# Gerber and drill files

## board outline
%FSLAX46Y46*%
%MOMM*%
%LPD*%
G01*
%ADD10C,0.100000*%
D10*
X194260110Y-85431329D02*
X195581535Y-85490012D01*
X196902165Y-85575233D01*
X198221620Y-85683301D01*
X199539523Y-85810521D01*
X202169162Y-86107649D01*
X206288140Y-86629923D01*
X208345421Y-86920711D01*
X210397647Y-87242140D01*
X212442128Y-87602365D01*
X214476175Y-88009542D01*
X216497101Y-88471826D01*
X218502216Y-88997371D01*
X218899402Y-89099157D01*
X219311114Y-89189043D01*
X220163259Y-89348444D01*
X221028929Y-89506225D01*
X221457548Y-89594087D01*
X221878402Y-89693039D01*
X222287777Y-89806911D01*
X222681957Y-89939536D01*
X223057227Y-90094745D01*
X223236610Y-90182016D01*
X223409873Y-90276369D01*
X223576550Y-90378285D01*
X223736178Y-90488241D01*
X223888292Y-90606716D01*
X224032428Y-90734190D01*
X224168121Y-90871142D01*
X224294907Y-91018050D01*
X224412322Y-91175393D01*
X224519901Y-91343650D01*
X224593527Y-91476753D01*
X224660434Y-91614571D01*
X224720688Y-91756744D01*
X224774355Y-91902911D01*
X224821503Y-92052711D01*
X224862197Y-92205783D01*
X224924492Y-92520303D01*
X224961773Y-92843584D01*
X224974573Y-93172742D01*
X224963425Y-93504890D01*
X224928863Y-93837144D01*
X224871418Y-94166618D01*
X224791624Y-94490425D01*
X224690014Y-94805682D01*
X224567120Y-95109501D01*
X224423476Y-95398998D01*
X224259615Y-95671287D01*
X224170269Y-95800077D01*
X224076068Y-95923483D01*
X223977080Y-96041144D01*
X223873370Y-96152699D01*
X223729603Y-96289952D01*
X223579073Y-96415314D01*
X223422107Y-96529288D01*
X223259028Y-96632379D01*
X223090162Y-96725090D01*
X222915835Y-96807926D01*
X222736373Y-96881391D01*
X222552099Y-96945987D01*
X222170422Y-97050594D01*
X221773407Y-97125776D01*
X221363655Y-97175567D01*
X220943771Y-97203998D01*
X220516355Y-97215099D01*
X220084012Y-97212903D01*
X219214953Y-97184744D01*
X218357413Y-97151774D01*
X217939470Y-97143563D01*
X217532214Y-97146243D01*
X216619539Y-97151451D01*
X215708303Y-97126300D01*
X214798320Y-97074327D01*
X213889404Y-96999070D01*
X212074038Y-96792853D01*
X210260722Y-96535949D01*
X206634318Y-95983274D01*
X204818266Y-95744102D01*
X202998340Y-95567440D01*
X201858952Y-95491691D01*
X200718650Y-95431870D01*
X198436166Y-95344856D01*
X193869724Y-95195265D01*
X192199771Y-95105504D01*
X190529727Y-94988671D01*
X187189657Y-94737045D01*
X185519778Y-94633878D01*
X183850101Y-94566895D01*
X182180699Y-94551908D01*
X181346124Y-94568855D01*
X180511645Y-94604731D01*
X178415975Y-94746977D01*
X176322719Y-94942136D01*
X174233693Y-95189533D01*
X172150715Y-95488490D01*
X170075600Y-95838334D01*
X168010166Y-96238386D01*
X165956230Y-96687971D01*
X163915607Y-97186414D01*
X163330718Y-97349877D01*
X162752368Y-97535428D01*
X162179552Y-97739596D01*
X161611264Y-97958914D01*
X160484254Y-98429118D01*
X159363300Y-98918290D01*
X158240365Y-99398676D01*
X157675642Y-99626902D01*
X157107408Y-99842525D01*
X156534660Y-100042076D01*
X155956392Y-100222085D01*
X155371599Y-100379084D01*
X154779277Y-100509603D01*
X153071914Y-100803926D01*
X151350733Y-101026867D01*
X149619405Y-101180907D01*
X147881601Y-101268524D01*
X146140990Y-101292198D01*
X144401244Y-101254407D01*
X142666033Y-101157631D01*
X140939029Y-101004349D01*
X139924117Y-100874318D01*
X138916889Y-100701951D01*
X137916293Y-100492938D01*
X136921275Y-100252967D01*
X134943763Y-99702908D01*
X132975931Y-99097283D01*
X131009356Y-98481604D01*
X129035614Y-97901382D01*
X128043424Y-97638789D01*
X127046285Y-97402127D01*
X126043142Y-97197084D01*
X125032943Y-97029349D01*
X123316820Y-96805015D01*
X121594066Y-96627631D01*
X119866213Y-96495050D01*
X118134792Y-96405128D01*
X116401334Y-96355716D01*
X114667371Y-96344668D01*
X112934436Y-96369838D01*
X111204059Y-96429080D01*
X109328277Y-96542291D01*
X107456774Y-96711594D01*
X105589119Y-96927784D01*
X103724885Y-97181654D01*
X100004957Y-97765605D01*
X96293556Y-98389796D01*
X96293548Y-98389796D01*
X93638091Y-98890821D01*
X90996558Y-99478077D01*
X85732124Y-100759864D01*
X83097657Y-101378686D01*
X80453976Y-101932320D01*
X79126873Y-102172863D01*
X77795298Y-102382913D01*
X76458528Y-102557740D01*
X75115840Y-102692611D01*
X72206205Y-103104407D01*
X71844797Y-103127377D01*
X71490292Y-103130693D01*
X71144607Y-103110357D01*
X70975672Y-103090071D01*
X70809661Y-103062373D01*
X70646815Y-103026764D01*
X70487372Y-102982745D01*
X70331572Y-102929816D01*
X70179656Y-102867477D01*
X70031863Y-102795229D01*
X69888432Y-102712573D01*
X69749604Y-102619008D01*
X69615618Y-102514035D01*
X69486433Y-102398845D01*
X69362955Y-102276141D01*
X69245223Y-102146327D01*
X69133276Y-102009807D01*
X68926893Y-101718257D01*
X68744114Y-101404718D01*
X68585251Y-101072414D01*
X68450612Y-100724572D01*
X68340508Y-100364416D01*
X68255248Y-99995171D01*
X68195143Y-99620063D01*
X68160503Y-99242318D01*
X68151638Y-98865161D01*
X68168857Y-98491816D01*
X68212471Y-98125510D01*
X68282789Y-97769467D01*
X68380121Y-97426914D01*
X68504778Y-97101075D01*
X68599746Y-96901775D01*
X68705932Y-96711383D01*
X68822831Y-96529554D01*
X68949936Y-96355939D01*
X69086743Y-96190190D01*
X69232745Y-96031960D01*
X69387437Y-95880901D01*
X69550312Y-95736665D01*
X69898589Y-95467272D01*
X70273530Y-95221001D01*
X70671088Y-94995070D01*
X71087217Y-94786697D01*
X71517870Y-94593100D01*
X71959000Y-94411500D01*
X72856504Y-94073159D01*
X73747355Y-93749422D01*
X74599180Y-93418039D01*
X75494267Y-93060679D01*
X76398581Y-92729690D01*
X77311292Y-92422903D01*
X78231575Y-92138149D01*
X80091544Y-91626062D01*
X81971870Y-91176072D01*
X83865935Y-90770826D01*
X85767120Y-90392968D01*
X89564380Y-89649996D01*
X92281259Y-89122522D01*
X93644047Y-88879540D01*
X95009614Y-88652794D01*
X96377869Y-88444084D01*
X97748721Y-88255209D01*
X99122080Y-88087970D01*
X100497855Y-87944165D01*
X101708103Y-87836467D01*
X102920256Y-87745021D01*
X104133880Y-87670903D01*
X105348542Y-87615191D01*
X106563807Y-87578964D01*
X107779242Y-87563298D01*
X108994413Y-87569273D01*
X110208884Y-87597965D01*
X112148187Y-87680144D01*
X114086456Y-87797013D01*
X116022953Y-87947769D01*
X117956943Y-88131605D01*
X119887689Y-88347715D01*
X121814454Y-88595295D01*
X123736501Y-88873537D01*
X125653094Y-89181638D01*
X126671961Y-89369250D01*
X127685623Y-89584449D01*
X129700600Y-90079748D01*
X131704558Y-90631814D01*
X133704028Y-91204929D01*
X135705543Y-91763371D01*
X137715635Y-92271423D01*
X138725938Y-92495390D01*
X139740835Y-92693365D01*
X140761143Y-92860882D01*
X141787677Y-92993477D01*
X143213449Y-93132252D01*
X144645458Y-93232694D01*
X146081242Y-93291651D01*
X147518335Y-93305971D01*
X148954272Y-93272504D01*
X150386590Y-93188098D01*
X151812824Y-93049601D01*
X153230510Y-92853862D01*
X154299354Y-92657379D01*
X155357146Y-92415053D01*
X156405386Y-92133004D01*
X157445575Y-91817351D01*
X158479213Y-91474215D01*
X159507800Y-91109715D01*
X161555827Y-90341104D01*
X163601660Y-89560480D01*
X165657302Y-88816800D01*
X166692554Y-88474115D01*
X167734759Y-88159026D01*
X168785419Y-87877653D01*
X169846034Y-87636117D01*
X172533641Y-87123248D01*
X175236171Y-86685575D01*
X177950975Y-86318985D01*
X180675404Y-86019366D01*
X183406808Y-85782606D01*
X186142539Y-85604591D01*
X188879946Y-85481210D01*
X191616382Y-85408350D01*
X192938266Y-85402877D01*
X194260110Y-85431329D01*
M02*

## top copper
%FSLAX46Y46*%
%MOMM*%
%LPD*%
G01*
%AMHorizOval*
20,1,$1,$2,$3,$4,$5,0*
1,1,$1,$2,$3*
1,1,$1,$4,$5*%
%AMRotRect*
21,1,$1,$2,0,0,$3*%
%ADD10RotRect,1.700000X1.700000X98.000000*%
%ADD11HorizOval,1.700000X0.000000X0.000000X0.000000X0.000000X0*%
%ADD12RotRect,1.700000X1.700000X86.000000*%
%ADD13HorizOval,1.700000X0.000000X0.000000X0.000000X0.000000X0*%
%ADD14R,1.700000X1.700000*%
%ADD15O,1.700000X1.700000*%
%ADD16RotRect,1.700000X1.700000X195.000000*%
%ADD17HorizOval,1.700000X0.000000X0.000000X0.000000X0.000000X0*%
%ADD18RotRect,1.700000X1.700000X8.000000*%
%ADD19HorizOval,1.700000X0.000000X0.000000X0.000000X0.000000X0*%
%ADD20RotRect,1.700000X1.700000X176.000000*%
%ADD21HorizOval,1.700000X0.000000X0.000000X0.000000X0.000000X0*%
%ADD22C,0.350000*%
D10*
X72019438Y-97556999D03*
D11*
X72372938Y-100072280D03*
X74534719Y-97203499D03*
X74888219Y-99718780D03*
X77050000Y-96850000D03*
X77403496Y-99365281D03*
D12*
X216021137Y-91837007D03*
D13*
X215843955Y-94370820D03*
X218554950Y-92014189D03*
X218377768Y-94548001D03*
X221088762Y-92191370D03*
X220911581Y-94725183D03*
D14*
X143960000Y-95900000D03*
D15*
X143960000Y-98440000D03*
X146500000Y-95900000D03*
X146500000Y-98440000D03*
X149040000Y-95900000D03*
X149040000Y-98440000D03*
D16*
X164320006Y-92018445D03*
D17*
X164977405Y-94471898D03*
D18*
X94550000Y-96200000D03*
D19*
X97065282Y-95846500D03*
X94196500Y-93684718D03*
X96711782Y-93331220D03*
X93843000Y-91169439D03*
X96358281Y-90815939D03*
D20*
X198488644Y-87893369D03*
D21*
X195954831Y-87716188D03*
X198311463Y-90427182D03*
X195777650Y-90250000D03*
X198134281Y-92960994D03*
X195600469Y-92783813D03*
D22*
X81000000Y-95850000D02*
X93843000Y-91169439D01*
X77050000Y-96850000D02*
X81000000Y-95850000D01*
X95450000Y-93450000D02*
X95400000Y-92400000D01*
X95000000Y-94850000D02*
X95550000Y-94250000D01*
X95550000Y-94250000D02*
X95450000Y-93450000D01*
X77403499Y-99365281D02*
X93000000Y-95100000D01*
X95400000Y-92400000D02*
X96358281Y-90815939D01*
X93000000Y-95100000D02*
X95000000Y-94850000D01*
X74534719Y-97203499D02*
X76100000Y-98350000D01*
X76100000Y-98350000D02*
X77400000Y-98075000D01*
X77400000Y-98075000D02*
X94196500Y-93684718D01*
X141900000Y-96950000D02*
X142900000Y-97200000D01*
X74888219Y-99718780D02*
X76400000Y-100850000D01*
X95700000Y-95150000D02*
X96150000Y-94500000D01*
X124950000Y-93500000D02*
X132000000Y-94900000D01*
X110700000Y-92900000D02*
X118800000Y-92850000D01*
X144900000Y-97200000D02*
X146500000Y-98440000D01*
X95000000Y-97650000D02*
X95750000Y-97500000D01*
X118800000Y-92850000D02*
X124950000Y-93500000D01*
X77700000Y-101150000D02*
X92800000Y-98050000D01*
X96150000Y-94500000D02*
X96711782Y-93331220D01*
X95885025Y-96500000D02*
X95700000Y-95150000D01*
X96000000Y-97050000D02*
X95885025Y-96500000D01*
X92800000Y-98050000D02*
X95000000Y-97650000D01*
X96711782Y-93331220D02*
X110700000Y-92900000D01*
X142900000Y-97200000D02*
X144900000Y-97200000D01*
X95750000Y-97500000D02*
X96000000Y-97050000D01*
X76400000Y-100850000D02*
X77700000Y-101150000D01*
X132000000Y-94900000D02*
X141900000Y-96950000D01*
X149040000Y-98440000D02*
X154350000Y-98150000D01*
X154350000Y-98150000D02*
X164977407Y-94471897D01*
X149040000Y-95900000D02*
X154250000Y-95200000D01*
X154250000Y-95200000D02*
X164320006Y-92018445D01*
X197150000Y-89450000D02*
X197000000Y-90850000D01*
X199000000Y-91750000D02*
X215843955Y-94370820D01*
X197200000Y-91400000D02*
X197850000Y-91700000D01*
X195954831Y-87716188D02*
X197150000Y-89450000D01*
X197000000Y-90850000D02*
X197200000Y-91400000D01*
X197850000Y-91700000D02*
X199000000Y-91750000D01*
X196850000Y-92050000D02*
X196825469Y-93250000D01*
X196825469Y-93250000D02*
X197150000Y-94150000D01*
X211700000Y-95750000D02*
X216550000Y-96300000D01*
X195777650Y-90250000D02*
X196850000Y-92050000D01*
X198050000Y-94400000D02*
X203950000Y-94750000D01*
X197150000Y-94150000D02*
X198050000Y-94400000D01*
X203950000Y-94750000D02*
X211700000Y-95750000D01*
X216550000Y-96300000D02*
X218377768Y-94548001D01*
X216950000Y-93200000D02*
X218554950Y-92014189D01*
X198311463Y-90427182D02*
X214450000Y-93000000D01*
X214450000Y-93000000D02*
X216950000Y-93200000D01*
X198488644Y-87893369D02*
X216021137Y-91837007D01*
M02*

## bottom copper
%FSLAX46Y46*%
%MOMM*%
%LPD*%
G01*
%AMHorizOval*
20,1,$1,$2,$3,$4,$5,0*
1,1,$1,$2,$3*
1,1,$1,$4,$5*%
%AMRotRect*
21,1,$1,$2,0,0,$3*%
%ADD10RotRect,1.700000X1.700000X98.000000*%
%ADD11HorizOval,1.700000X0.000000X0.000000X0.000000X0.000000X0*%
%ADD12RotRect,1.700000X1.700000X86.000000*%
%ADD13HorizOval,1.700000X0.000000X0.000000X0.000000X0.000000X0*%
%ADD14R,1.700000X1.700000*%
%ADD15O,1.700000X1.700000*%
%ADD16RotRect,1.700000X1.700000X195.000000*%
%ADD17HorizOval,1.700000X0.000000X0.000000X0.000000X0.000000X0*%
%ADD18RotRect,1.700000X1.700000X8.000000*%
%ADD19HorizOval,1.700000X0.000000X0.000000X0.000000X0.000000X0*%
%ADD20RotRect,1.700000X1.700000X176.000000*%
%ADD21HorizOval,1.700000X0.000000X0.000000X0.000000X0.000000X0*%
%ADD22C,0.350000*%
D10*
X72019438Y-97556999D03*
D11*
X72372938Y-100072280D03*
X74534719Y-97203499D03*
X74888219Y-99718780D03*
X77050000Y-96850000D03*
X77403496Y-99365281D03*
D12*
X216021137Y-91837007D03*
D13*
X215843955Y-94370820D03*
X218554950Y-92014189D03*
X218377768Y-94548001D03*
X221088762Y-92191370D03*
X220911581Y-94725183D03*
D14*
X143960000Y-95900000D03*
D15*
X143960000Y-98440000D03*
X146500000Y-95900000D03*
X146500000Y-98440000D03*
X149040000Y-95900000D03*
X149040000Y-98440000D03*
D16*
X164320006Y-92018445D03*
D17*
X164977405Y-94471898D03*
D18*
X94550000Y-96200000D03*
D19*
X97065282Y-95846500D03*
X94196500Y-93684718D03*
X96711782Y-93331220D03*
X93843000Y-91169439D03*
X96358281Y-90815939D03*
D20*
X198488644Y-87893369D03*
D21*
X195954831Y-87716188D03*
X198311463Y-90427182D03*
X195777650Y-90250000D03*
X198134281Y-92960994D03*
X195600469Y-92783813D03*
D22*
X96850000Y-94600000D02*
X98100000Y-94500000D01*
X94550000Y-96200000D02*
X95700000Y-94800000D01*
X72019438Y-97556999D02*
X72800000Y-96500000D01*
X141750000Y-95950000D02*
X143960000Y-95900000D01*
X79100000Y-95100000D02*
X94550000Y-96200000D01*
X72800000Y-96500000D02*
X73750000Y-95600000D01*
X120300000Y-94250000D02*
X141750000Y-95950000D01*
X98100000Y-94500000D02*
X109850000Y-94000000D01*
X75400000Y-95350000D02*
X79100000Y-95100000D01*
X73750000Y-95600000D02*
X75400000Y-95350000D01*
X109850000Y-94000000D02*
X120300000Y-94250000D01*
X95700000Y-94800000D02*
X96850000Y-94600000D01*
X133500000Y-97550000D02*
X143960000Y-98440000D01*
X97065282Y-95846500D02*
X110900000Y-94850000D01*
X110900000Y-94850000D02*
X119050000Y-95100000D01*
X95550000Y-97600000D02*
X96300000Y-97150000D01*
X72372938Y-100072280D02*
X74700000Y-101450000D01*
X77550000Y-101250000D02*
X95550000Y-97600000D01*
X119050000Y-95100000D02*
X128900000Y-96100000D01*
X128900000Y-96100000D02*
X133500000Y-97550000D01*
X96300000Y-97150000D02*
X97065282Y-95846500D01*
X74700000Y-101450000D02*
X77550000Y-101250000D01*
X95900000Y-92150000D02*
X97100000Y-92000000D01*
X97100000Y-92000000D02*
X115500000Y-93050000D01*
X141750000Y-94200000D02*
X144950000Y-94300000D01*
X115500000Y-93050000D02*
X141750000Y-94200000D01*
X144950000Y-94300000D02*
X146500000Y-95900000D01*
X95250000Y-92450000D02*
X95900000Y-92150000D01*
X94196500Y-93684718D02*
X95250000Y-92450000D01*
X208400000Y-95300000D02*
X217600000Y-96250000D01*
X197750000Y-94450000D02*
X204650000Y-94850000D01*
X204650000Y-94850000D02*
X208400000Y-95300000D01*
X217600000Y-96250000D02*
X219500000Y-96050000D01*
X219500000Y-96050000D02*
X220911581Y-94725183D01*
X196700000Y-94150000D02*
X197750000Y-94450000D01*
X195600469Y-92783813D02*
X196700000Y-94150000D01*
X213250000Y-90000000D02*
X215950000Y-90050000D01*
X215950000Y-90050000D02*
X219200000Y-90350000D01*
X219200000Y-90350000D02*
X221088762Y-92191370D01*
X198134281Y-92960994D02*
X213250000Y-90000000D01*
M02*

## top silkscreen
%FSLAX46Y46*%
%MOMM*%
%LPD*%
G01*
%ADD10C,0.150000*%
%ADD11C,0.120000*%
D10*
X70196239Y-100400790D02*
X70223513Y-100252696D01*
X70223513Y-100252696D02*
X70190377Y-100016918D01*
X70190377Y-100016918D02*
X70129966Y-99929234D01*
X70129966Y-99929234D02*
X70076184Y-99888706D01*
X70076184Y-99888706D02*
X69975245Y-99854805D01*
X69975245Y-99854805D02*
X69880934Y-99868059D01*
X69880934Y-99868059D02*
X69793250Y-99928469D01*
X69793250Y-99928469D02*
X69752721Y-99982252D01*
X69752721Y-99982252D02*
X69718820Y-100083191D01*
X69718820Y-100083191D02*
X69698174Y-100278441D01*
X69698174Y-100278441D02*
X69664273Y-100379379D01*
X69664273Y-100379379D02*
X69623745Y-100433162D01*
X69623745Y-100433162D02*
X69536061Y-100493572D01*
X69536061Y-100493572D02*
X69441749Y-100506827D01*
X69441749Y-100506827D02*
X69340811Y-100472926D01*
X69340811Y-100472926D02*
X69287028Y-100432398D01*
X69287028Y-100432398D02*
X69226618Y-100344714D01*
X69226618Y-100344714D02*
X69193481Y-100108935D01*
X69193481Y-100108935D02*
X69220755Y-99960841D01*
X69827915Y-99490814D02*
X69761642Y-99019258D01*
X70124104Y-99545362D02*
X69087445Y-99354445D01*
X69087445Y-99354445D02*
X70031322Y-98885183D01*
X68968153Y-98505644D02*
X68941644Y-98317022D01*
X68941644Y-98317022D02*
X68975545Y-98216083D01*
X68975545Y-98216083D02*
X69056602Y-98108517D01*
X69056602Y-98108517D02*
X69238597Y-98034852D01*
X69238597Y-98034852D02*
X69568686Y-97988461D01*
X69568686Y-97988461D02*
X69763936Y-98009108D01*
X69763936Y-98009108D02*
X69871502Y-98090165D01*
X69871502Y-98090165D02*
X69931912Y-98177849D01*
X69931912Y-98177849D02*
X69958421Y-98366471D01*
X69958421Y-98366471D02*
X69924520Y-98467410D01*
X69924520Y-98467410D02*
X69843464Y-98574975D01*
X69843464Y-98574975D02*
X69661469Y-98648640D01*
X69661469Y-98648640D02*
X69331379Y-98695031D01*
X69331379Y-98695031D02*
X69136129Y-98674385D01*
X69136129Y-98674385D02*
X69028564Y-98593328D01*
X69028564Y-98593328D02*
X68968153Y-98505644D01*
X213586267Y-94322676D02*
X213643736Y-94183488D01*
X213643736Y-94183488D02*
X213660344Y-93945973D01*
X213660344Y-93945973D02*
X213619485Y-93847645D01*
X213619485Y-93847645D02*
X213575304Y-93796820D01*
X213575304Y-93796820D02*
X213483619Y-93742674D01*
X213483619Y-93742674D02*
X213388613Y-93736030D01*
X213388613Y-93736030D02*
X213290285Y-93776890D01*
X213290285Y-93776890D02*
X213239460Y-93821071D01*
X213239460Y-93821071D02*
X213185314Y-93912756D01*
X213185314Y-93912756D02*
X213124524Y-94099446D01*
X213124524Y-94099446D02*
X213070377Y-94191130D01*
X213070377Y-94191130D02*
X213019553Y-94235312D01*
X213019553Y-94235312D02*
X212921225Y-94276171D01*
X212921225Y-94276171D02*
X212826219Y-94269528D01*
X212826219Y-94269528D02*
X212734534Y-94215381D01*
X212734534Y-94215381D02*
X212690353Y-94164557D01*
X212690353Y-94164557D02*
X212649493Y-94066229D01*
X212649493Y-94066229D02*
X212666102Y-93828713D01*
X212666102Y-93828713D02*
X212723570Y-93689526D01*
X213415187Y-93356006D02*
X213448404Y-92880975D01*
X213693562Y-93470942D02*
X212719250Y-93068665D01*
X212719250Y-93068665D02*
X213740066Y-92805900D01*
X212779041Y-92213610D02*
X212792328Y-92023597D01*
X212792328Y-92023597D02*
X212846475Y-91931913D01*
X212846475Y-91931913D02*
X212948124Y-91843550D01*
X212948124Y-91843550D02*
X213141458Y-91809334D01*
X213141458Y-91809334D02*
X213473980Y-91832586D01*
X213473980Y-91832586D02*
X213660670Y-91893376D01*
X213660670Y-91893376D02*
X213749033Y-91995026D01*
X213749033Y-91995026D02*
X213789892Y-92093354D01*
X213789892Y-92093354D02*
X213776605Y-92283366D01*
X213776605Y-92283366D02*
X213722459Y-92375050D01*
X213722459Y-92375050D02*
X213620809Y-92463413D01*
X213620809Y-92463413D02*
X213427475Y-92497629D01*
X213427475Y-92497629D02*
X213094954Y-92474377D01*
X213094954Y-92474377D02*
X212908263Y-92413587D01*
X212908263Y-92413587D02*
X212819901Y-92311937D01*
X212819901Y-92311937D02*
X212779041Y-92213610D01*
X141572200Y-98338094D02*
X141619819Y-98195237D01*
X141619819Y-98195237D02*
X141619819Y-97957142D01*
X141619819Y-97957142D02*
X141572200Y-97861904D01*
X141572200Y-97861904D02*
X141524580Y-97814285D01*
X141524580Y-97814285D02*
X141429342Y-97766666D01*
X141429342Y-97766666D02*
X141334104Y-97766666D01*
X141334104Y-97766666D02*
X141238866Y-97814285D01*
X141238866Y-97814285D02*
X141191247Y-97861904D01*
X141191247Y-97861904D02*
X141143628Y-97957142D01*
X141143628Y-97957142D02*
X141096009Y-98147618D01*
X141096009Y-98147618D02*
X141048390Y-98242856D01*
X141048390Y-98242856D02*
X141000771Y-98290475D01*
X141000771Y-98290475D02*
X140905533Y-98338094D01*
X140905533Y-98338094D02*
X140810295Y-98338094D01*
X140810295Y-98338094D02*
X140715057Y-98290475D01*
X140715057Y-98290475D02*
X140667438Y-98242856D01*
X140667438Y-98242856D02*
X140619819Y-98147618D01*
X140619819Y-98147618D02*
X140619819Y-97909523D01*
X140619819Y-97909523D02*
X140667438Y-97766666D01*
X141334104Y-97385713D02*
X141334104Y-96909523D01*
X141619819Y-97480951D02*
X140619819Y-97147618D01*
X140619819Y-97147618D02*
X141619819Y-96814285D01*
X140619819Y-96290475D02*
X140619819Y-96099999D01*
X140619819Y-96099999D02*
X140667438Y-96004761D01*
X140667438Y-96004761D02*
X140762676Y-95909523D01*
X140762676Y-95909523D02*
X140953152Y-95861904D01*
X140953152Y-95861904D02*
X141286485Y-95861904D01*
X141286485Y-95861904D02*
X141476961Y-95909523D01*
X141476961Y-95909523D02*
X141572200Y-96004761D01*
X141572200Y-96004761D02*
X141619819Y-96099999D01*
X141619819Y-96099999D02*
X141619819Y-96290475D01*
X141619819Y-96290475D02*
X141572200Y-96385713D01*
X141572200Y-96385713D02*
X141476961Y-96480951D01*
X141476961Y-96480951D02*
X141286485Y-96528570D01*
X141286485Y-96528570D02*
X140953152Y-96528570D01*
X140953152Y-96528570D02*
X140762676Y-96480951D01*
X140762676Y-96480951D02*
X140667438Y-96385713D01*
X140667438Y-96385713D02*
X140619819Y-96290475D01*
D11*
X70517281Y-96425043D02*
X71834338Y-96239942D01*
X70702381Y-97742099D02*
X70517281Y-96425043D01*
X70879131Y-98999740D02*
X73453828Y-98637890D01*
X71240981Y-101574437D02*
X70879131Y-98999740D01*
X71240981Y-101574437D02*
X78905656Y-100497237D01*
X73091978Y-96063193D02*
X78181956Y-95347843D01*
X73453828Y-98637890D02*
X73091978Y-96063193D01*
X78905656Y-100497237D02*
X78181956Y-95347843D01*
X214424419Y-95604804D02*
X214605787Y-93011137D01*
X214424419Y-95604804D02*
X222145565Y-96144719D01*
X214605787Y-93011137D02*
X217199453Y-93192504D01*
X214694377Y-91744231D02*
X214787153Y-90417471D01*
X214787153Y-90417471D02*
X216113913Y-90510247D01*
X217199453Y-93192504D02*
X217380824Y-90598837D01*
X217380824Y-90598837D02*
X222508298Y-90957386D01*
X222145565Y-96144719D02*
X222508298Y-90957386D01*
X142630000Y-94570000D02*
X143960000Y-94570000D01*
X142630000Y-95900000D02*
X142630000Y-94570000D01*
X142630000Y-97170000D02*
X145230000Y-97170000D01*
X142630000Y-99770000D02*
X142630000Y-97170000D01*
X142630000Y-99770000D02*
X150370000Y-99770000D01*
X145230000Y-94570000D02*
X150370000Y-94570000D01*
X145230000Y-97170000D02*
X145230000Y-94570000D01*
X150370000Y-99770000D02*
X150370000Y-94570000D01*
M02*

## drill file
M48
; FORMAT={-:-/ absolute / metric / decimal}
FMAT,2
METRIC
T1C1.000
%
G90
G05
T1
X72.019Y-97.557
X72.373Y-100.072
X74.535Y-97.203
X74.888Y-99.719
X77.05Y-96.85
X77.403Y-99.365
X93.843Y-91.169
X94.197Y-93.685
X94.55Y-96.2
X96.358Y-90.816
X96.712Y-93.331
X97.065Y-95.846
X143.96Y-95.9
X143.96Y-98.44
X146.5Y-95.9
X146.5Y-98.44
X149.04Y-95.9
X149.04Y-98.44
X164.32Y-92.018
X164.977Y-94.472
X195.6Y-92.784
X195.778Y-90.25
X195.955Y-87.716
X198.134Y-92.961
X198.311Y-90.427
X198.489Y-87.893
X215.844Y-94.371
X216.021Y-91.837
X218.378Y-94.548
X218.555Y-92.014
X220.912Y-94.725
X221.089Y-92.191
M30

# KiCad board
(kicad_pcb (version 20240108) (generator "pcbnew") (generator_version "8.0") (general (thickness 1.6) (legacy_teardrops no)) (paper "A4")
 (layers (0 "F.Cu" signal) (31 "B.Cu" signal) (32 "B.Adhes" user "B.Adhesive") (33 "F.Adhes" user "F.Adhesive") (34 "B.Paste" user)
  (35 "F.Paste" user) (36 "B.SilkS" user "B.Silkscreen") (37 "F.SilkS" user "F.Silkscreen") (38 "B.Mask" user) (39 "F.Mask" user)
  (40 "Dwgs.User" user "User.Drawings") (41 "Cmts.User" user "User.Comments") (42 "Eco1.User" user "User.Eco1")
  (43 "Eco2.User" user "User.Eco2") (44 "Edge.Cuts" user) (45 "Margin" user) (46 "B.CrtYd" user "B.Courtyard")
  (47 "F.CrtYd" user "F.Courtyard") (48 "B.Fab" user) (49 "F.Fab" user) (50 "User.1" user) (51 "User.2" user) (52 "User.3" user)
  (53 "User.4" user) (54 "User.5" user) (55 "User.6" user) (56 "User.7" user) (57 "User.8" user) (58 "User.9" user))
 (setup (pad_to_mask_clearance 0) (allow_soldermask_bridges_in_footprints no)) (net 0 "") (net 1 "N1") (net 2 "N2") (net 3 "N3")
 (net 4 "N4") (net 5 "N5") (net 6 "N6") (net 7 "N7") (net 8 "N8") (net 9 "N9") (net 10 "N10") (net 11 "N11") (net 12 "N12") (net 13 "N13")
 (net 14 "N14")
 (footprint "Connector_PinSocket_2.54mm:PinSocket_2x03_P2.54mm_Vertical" (layer "F.Cu") (at 72.019438 97.556999 98)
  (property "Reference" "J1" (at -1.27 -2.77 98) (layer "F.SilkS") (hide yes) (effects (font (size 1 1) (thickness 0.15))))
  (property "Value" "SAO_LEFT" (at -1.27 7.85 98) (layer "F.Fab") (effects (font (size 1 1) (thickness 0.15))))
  (fp_line (start 1.33 -1.33) (end 1.33 0) (stroke (width 0.12) (type solid)) (layer "F.SilkS"))
  (fp_line (start 0 -1.33) (end 1.33 -1.33) (stroke (width 0.12) (type solid)) (layer "F.SilkS"))
  (fp_line (start -1.27 -1.33) (end -1.27 1.27) (stroke (width 0.12) (type solid)) (layer "F.SilkS"))
  (fp_line (start -3.87 -1.33) (end -1.27 -1.33) (stroke (width 0.12) (type solid)) (layer "F.SilkS"))
  (fp_line (start -3.87 -1.33) (end -3.87 6.41) (stroke (width 0.12) (type solid)) (layer "F.SilkS"))
  (fp_line (start 1.33 1.27) (end 1.33 6.41) (stroke (width 0.12) (type solid)) (layer "F.SilkS"))
  (fp_line (start -1.27 1.27) (end 1.33 1.27) (stroke (width 0.12) (type solid)) (layer "F.SilkS"))
  (fp_line (start -3.87 6.41) (end 1.33 6.41) (stroke (width 0.12) (type solid)) (layer "F.SilkS"))
  (pad "1" thru_hole rect (at 0 0 98) (size 1.7 1.7) (drill 1) (layers "*.Cu" "*.Mask") (remove_unused_layers no) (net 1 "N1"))
  (pad "2" thru_hole oval (at -2.54 0 98) (size 1.7 1.7) (drill 1) (layers "*.Cu" "*.Mask") (remove_unused_layers no) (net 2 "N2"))
  (pad "3" thru_hole oval (at 0 2.54 98) (size 1.7 1.7) (drill 1) (layers "*.Cu" "*.Mask") (remove_unused_layers no) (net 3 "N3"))
  (pad "4" thru_hole oval (at -2.54 2.54 98) (size 1.7 1.7) (drill 1) (layers "*.Cu" "*.Mask") (remove_unused_layers no) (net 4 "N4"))
  (pad "5" thru_hole oval (at 0 5.08 98) (size 1.7 1.7) (drill 1) (layers "*.Cu" "*.Mask") (remove_unused_layers no) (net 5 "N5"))
  (pad "6" thru_hole oval (at -2.54 5.079997 98) (size 1.7 1.7) (drill 1) (layers "*.Cu" "*.Mask") (remove_unused_layers no) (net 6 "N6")))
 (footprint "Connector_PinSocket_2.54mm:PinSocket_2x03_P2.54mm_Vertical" (layer "F.Cu") (at 216.021137 91.837007 86)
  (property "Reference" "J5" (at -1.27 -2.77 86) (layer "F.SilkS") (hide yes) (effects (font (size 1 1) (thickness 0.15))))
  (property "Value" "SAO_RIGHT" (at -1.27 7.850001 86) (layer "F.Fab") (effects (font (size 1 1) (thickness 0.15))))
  (fp_line (start -3.87 -1.33) (end -1.27 -1.329999) (stroke (width 0.12) (type solid)) (layer "F.SilkS"))
  (fp_line (start -3.87 -1.33) (end -3.87 6.41) (stroke (width 0.12) (type solid)) (layer "F.SilkS"))
  (fp_line (start -1.27 -1.329999) (end -1.27 1.27) (stroke (width 0.12) (type solid)) (layer "F.SilkS"))
  (fp_line (start 0 -1.33) (end 1.33 -1.33) (stroke (width 0.12) (type solid)) (layer "F.SilkS"))
  (fp_line (start 1.33 -1.33) (end 1.33 0) (stroke (width 0.12) (type solid)) (layer "F.SilkS"))
  (fp_line (start -1.27 1.27) (end 1.330001 1.270004) (stroke (width 0.12) (type solid)) (layer "F.SilkS"))
  (fp_line (start 1.330001 1.270004) (end 1.33 6.409999) (stroke (width 0.12) (type solid)) (layer "F.SilkS"))
  (fp_line (start -3.87 6.41) (end 1.33 6.409999) (stroke (width 0.12) (type solid)) (layer "F.SilkS"))
  (pad "1" thru_hole rect (at 0 0 86) (size 1.7 1.7) (drill 1) (layers "*.Cu" "*.Mask") (remove_unused_layers no) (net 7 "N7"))
  (pad "2" thru_hole oval (at -2.54 -0.000001 86) (size 1.7 1.7) (drill 1) (layers "*.Cu" "*.Mask") (remove_unused_layers no) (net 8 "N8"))
  (pad "3" thru_hole oval (at -0.000001 2.54 86) (size 1.7 1.7) (drill 1) (layers "*.Cu" "*.Mask") (remove_unused_layers no) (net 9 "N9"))
  (pad "4" thru_hole oval (at -2.54 2.54 86) (size 1.7 1.7) (drill 1) (layers "*.Cu" "*.Mask") (remove_unused_layers no) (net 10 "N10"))
  (pad "5" thru_hole oval (at 0 5.08 86) (size 1.7 1.7) (drill 1) (layers "*.Cu" "*.Mask") (remove_unused_layers no) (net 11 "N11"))
  (pad "6" thru_hole oval (at -2.54 5.08 86) (size 1.7 1.7) (drill 1) (layers "*.Cu" "*.Mask") (remove_unused_layers no) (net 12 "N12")))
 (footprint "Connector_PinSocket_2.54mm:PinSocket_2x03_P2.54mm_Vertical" (layer "F.Cu") (at 143.96 95.9 90)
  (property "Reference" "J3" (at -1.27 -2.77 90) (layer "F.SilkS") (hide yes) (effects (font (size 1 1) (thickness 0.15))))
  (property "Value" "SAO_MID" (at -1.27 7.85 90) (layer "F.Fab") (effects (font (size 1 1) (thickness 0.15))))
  (fp_line (start 1.33 -1.33) (end 1.33 0) (stroke (width 0.12) (type solid)) (layer "F.SilkS"))
  (fp_line (start 0 -1.33) (end 1.33 -1.33) (stroke (width 0.12) (type solid)) (layer "F.SilkS"))
  (fp_line (start -1.27 -1.33) (end -1.27 1.27) (stroke (width 0.12) (type solid)) (layer "F.SilkS"))
  (fp_line (start -3.87 -1.33) (end -1.27 -1.33) (stroke (width 0.12) (type solid)) (layer "F.SilkS"))
  (fp_line (start -3.87 -1.33) (end -3.87 6.41) (stroke (width 0.12) (type solid)) (layer "F.SilkS"))
  (fp_line (start 1.33 1.27) (end 1.33 6.41) (stroke (width 0.12) (type solid)) (layer "F.SilkS"))
  (fp_line (start -1.27 1.27) (end 1.33 1.27) (stroke (width 0.12) (type solid)) (layer "F.SilkS"))
  (fp_line (start -3.87 6.41) (end 1.33 6.41) (stroke (width 0.12) (type solid)) (layer "F.SilkS"))
  (pad "1" thru_hole rect (at 0 0 90) (size 1.7 1.7) (drill 1) (layers "*.Cu" "*.Mask") (remove_unused_layers no) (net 1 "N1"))
  (pad "2" thru_hole oval (at -2.54 0 90) (size 1.7 1.7) (drill 1) (layers "*.Cu" "*.Mask") (remove_unused_layers no) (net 2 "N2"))
  (pad "3" thru_hole oval (at 0 2.54 90) (size 1.7 1.7) (drill 1) (layers "*.Cu" "*.Mask") (remove_unused_layers no) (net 3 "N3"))
  (pad "4" thru_hole oval (at -2.54 2.54 90) (size 1.7 1.7) (drill 1) (layers "*.Cu" "*.Mask") (remove_unused_layers no) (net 4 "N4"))
  (pad "5" thru_hole oval (at 0 5.08 90) (size 1.7 1.7) (drill 1) (layers "*.Cu" "*.Mask") (remove_unused_layers no) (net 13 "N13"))
  (pad "6" thru_hole oval (at -2.54 5.08 90) (size 1.7 1.7) (drill 1) (layers "*.Cu" "*.Mask") (remove_unused_layers no) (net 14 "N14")))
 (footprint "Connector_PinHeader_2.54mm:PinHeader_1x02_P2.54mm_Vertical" (layer "B.Cu") (at 164.320006 92.018445 -165)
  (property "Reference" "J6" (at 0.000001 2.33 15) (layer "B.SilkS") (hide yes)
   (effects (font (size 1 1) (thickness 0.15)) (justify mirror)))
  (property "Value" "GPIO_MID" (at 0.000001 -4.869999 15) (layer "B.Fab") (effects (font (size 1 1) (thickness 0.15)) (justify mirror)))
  (pad "1" thru_hole rect (at 0 0 195) (size 1.7 1.7) (drill 1) (layers "*.Cu" "*.Mask") (remove_unused_layers no) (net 13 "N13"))
  (pad "2" thru_hole oval (at 0.000002 -2.540001 195) (size 1.7 1.7) (drill 1) (layers "*.Cu" "*.Mask") (remove_unused_layers no)
   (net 14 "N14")))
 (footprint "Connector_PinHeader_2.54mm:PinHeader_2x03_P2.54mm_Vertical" (layer "B.Cu") (at 94.55 96.2 8)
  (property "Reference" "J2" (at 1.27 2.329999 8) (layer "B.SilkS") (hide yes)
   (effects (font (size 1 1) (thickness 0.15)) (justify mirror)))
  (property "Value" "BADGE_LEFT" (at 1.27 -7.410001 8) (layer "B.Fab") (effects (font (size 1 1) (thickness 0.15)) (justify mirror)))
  (pad "1" thru_hole rect (at 0 0 8) (size 1.7 1.7) (drill 1) (layers "*.Cu" "*.Mask") (remove_unused_layers no) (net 1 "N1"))
  (pad "2" thru_hole oval (at 2.540001 0 8) (size 1.7 1.7) (drill 1) (layers "*.Cu" "*.Mask") (remove_unused_layers no) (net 2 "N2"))
  (pad "3" thru_hole oval (at 0 -2.540001 8) (size 1.7 1.7) (drill 1) (layers "*.Cu" "*.Mask") (remove_unused_layers no) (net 3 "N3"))
  (pad "4" thru_hole oval (at 2.540001 -2.539999 8) (size 1.7 1.7) (drill 1) (layers "*.Cu" "*.Mask") (remove_unused_layers no) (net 4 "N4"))
  (pad "5" thru_hole oval (at -0.000001 -5.079999 8) (size 1.7 1.7) (drill 1) (layers "*.Cu" "*.Mask") (remove_unused_layers no)
   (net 5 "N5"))
  (pad "6" thru_hole oval (at 2.539999 -5.08 8) (size 1.7 1.7) (drill 1) (layers "*.Cu" "*.Mask") (remove_unused_layers no) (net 6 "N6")))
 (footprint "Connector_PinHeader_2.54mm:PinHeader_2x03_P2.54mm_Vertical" (layer "B.Cu") (at 198.488644 87.893369 176)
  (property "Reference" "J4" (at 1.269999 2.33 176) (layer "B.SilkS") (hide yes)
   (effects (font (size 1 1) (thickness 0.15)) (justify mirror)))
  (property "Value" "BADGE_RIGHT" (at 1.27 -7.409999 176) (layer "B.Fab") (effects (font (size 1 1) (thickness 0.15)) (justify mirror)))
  (pad "1" thru_hole rect (at 0 0 176) (size 1.7 1.7) (drill 1) (layers "*.Cu" "*.Mask") (remove_unused_layers no) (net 7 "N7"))
  (pad "2" thru_hole oval (at 2.54 0 176) (size 1.7 1.7) (drill 1) (layers "*.Cu" "*.Mask") (remove_unused_layers no) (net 8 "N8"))
  (pad "3" thru_hole oval (at 0 -2.54 176) (size 1.7 1.7) (drill 1) (layers "*.Cu" "*.Mask") (remove_unused_layers no) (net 9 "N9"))
  (pad "4" thru_hole oval (at 2.54 -2.54 176) (size 1.7 1.7) (drill 1) (layers "*.Cu" "*.Mask") (remove_unused_layers no) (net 10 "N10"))
  (pad "5" thru_hole oval (at 0 -5.08 176) (size 1.7 1.7) (drill 1) (layers "*.Cu" "*.Mask") (remove_unused_layers no) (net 11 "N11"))
  (pad "6" thru_hole oval (at 2.539999 -5.08 176) (size 1.7 1.7) (drill 1) (layers "*.Cu" "*.Mask") (remove_unused_layers no) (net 12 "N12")))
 (gr_poly
  (pts (xy 194.26011 85.431329) (xy 195.581535 85.490012) (xy 196.902165 85.575233) (xy 198.22162 85.683301) (xy 199.539523 85.810521)
   (xy 202.169162 86.107649) (xy 206.28814 86.629923) (xy 208.345421 86.920711) (xy 210.397647 87.24214) (xy 212.442128 87.602365)
   (xy 214.476175 88.009542) (xy 216.497101 88.471826) (xy 218.502216 88.997371) (xy 218.899402 89.099157) (xy 219.311114 89.189043)
   (xy 220.163259 89.348444) (xy 221.028929 89.506225) (xy 221.457548 89.594087) (xy 221.878402 89.693039) (xy 222.287777 89.806911)
   (xy 222.681957 89.939536) (xy 223.057227 90.094745) (xy 223.23661 90.182016) (xy 223.409873 90.276369) (xy 223.57655 90.378285)
   (xy 223.736178 90.488241) (xy 223.888292 90.606716) (xy 224.032428 90.73419) (xy 224.168121 90.871142) (xy 224.294907 91.01805)
   (xy 224.412322 91.175393) (xy 224.519901 91.34365) (xy 224.593527 91.476753) (xy 224.660434 91.614571) (xy 224.720688 91.756744)
   (xy 224.774355 91.902911) (xy 224.821503 92.052711) (xy 224.862197 92.205783) (xy 224.924492 92.520303) (xy 224.961773 92.843584)
   (xy 224.974573 93.172742) (xy 224.963425 93.50489) (xy 224.928863 93.837144) (xy 224.871418 94.166618) (xy 224.791624 94.490425)
   (xy 224.690014 94.805682) (xy 224.56712 95.109501) (xy 224.423476 95.398998) (xy 224.259615 95.671287) (xy 224.170269 95.800077)
   (xy 224.076068 95.923483) (xy 223.97708 96.041144) (xy 223.87337 96.152699) (xy 223.729603 96.289952) (xy 223.579073 96.415314)
   (xy 223.422107 96.529288) (xy 223.259028 96.632379) (xy 223.090162 96.72509) (xy 222.915835 96.807926) (xy 222.736373 96.881391)
   (xy 222.552099 96.945987) (xy 222.170422 97.050594) (xy 221.773407 97.125776) (xy 221.363655 97.175567) (xy 220.943771 97.203998)
   (xy 220.516355 97.215099) (xy 220.084012 97.212903) (xy 219.214953 97.184744) (xy 218.357413 97.151774) (xy 217.93947 97.143563)
   (xy 217.532214 97.146243) (xy 216.619539 97.151451) (xy 215.708303 97.1263) (xy 214.79832 97.074327) (xy 213.889404 96.99907)
   (xy 212.074038 96.792853) (xy 210.260722 96.535949) (xy 206.634318 95.983274) (xy 204.818266 95.744102) (xy 202.99834 95.56744)
   (xy 201.858952 95.491691) (xy 200.71865 95.43187) (xy 198.436166 95.344856) (xy 193.869724 95.195265) (xy 192.199771 95.105504)
   (xy 190.529727 94.988671) (xy 187.189657 94.737045) (xy 185.519778 94.633878) (xy 183.850101 94.566895) (xy 182.180699 94.551908)
   (xy 181.346124 94.568855) (xy 180.511645 94.604731) (xy 178.415975 94.746977) (xy 176.322719 94.942136) (xy 174.233693 95.189533)
   (xy 172.150715 95.48849) (xy 170.0756 95.838334) (xy 168.010166 96.238386) (xy 165.95623 96.687971) (xy 163.915607 97.186414)
   (xy 163.330718 97.349877) (xy 162.752368 97.535428) (xy 162.179552 97.739596) (xy 161.611264 97.958914) (xy 160.484254 98.429118)
   (xy 159.3633 98.91829) (xy 158.240365 99.398676) (xy 157.675642 99.626902) (xy 157.107408 99.842525) (xy 156.53466 100.042076)
   (xy 155.956392 100.222085) (xy 155.371599 100.379084) (xy 154.779277 100.509603) (xy 153.071914 100.803926) (xy 151.350733 101.026867)
   (xy 149.619405 101.180907) (xy 147.881601 101.268524) (xy 146.14099 101.292198) (xy 144.401244 101.254407) (xy 142.666033 101.157631)
   (xy 140.939029 101.004349) (xy 139.924117 100.874318) (xy 138.916889 100.701951) (xy 137.916293 100.492938) (xy 136.921275 100.252967)
   (xy 134.943763 99.702908) (xy 132.975931 99.097283) (xy 131.009356 98.481604) (xy 129.035614 97.901382) (xy 128.043424 97.638789)
   (xy 127.046285 97.402127) (xy 126.043142 97.197084) (xy 125.032943 97.029349) (xy 123.31682 96.805015) (xy 121.594066 96.627631)
   (xy 119.866213 96.49505) (xy 118.134792 96.405128) (xy 116.401334 96.355716) (xy 114.667371 96.344668) (xy 112.934436 96.369838)
   (xy 111.204059 96.42908) (xy 109.328277 96.542291) (xy 107.456774 96.711594) (xy 105.589119 96.927784) (xy 103.724885 97.181654)
   (xy 100.004957 97.765605) (xy 96.293556 98.389796) (xy 96.293548 98.389796) (xy 93.638091 98.890821) (xy 90.996558 99.478077)
   (xy 85.732124 100.759864) (xy 83.097657 101.378686) (xy 80.453976 101.93232) (xy 79.126873 102.172863) (xy 77.795298 102.382913)
   (xy 76.458528 102.55774) (xy 75.11584 102.692611) (xy 72.206205 103.104407) (xy 71.844797 103.127377) (xy 71.490292 103.130693)
   (xy 71.144607 103.110357) (xy 70.975672 103.090071) (xy 70.809661 103.062373) (xy 70.646815 103.026764) (xy 70.487372 102.982745)
   (xy 70.331572 102.929816) (xy 70.179656 102.867477) (xy 70.031863 102.795229) (xy 69.888432 102.712573) (xy 69.749604 102.619008)
   (xy 69.615618 102.514035) (xy 69.486433 102.398845) (xy 69.362955 102.276141) (xy 69.245223 102.146327) (xy 69.133276 102.009807)
   (xy 68.926893 101.718257) (xy 68.744114 101.404718) (xy 68.585251 101.072414) (xy 68.450612 100.724572) (xy 68.340508 100.364416)
   (xy 68.255248 99.995171) (xy 68.195143 99.620063) (xy 68.160503 99.242318) (xy 68.151638 98.865161) (xy 68.168857 98.491816)
   (xy 68.212471 98.12551) (xy 68.282789 97.769467) (xy 68.380121 97.426914) (xy 68.504778 97.101075) (xy 68.599746 96.901775)
   (xy 68.705932 96.711383) (xy 68.822831 96.529554) (xy 68.949936 96.355939) (xy 69.086743 96.19019) (xy 69.232745 96.03196)
   (xy 69.387437 95.880901) (xy 69.550312 95.736665) (xy 69.898589 95.467272) (xy 70.27353 95.221001) (xy 70.671088 94.99507)
   (xy 71.087217 94.786697) (xy 71.51787 94.5931) (xy 71.959 94.4115) (xy 72.856504 94.073159) (xy 73.747355 93.749422)
   (xy 74.59918 93.418039) (xy 75.494267 93.060679) (xy 76.398581 92.72969) (xy 77.311292 92.422903) (xy 78.231575 92.138149)
   (xy 80.091544 91.626062) (xy 81.97187 91.176072) (xy 83.865935 90.770826) (xy 85.76712 90.392968) (xy 89.56438 89.649996)
   (xy 92.281259 89.122522) (xy 93.644047 88.87954) (xy 95.009614 88.652794) (xy 96.377869 88.444084) (xy 97.748721 88.255209)
   (xy 99.12208 88.08797) (xy 100.497855 87.944165) (xy 101.708103 87.836467) (xy 102.920256 87.745021) (xy 104.13388 87.670903)
   (xy 105.348542 87.615191) (xy 106.563807 87.578964) (xy 107.779242 87.563298) (xy 108.994413 87.569273) (xy 110.208884 87.597965)
   (xy 112.148187 87.680144) (xy 114.086456 87.797013) (xy 116.022953 87.947769) (xy 117.956943 88.131605) (xy 119.887689 88.347715)
   (xy 121.814454 88.595295) (xy 123.736501 88.873537) (xy 125.653094 89.181638) (xy 126.671961 89.36925) (xy 127.685623 89.584449)
   (xy 129.7006 90.079748) (xy 131.704558 90.631814) (xy 133.704028 91.204929) (xy 135.705543 91.763371) (xy 137.715635 92.271423)
   (xy 138.725938 92.49539) (xy 139.740835 92.693365) (xy 140.761143 92.860882) (xy 141.787677 92.993477) (xy 143.213449 93.132252)
   (xy 144.645458 93.232694) (xy 146.081242 93.291651) (xy 147.518335 93.305971) (xy 148.954272 93.272504) (xy 150.38659 93.188098)
   (xy 151.812824 93.049601) (xy 153.23051 92.853862) (xy 154.299354 92.657379) (xy 155.357146 92.415053) (xy 156.405386 92.133004)
   (xy 157.445575 91.817351) (xy 158.479213 91.474215) (xy 159.5078 91.109715) (xy 161.555827 90.341104) (xy 163.60166 89.56048)
   (xy 165.657302 88.8168) (xy 166.692554 88.474115) (xy 167.734759 88.159026) (xy 168.785419 87.877653) (xy 169.846034 87.636117)
   (xy 172.533641 87.123248) (xy 175.236171 86.685575) (xy 177.950975 86.318985) (xy 180.675404 86.019366) (xy 183.406808 85.782606)
   (xy 186.142539 85.604591) (xy 188.879946 85.48121) (xy 191.616382 85.40835) (xy 192.938266 85.402877))
  (stroke (width 0.1) (type solid)) (fill none) (layer "Edge.Cuts"))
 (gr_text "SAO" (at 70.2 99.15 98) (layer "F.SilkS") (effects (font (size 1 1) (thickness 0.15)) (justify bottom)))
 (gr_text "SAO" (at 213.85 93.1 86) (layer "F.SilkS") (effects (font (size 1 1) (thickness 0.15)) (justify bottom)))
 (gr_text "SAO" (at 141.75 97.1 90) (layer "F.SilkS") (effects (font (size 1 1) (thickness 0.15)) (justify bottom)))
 (segment (start 96.85 94.6) (end 98.1 94.5) (width 0.35) (layer "B.Cu") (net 1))
 (segment (start 94.55 96.2) (end 95.7 94.8) (width 0.35) (layer "B.Cu") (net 1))
 (segment (start 72.019438 97.556999) (end 72.8 96.5) (width 0.35) (layer "B.Cu") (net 1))
 (segment (start 141.75 95.95) (end 143.96 95.9) (width 0.35) (layer "B.Cu") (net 1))
 (segment (start 79.1 95.1) (end 94.55 96.2) (width 0.35) (layer "B.Cu") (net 1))
 (segment (start 72.8 96.5) (end 73.75 95.6) (width 0.35) (layer "B.Cu") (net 1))
 (segment (start 120.3 94.25) (end 141.75 95.95) (width 0.35) (layer "B.Cu") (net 1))
 (segment (start 98.1 94.5) (end 109.85 94) (width 0.35) (layer "B.Cu") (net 1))
 (segment (start 75.4 95.35) (end 79.1 95.1) (width 0.35) (layer "B.Cu") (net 1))
 (segment (start 73.75 95.6) (end 75.4 95.35) (width 0.35) (layer "B.Cu") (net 1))
 (segment (start 109.85 94) (end 120.3 94.25) (width 0.35) (layer "B.Cu") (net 1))
 (segment (start 95.7 94.8) (end 96.85 94.6) (width 0.35) (layer "B.Cu") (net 1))
 (segment (start 81 95.85) (end 93.843 91.169439) (width 0.35) (layer "F.Cu") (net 5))
 (segment (start 77.05 96.85) (end 81 95.85) (width 0.35) (layer "F.Cu") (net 5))
 (segment (start 95.45 93.45) (end 95.4 92.4) (width 0.35) (layer "F.Cu") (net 6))
 (segment (start 95 94.85) (end 95.55 94.25) (width 0.35) (layer "F.Cu") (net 6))
 (segment (start 95.55 94.25) (end 95.45 93.45) (width 0.35) (layer "F.Cu") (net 6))
 (segment (start 77.403499 99.365281) (end 93 95.1) (width 0.35) (layer "F.Cu") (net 6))
 (segment (start 95.4 92.4) (end 96.358281 90.815939) (width 0.35) (layer "F.Cu") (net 6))
 (segment (start 93 95.1) (end 95 94.85) (width 0.35) (layer "F.Cu") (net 6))
 (segment (start 133.5 97.55) (end 143.96 98.44) (width 0.35) (layer "B.Cu") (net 2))
 (segment (start 97.065282 95.8465) (end 110.9 94.85) (width 0.35) (layer "B.Cu") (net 2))
 (segment (start 110.9 94.85) (end 119.05 95.1) (width 0.35) (layer "B.Cu") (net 2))
 (segment (start 95.55 97.6) (end 96.3 97.15) (width 0.35) (layer "B.Cu") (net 2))
 (segment (start 72.372938 100.07228) (end 74.7 101.45) (width 0.35) (layer "B.Cu") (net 2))
 (segment (start 77.55 101.25) (end 95.55 97.6) (width 0.35) (layer "B.Cu") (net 2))
 (segment (start 119.05 95.1) (end 128.9 96.1) (width 0.35) (layer "B.Cu") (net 2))
 (segment (start 128.9 96.1) (end 133.5 97.55) (width 0.35) (layer "B.Cu") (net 2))
 (segment (start 96.3 97.15) (end 97.065282 95.8465) (width 0.35) (layer "B.Cu") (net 2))
 (segment (start 74.7 101.45) (end 77.55 101.25) (width 0.35) (layer "B.Cu") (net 2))
 (segment (start 74.534719 97.203499) (end 76.1 98.35) (width 0.35) (layer "F.Cu") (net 3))
 (segment (start 76.1 98.35) (end 77.4 98.075) (width 0.35) (layer "F.Cu") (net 3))
 (segment (start 77.4 98.075) (end 94.1965 93.684718) (width 0.35) (layer "F.Cu") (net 3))
 (segment (start 95.9 92.15) (end 97.1 92) (width 0.35) (layer "B.Cu") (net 3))
 (segment (start 97.1 92) (end 115.5 93.05) (width 0.35) (layer "B.Cu") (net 3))
 (segment (start 141.75 94.2) (end 144.95 94.3) (width 0.35) (layer "B.Cu") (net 3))
 (segment (start 115.5 93.05) (end 141.75 94.2) (width 0.35) (layer "B.Cu") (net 3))
 (segment (start 144.95 94.3) (end 146.5 95.9) (width 0.35) (layer "B.Cu") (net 3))
 (segment (start 95.25 92.45) (end 95.9 92.15) (width 0.35) (layer "B.Cu") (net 3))
 (segment (start 94.1965 93.684718) (end 95.25 92.45) (width 0.35) (layer "B.Cu") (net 3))
 (segment (start 141.9 96.95) (end 142.9 97.2) (width 0.35) (layer "F.Cu") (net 4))
 (segment (start 74.888219 99.71878) (end 76.4 100.85) (width 0.35) (layer "F.Cu") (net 4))
 (segment (start 95.7 95.15) (end 96.15 94.5) (width 0.35) (layer "F.Cu") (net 4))
 (segment (start 124.95 93.5) (end 132 94.9) (width 0.35) (layer "F.Cu") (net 4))
 (segment (start 110.7 92.9) (end 118.8 92.85) (width 0.35) (layer "F.Cu") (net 4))
 (segment (start 144.9 97.2) (end 146.5 98.44) (width 0.35) (layer "F.Cu") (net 4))
 (segment (start 95 97.65) (end 95.75 97.5) (width 0.35) (layer "F.Cu") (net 4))
 (segment (start 118.8 92.85) (end 124.95 93.5) (width 0.35) (layer "F.Cu") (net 4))
 (segment (start 77.7 101.15) (end 92.8 98.05) (width 0.35) (layer "F.Cu") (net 4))
 (segment (start 96.15 94.5) (end 96.711782 93.33122) (width 0.35) (layer "F.Cu") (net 4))
 (segment (start 95.885025 96.5) (end 95.7 95.15) (width 0.35) (layer "F.Cu") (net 4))
 (segment (start 96 97.05) (end 95.885025 96.5) (width 0.35) (layer "F.Cu") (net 4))
 (segment (start 92.8 98.05) (end 95 97.65) (width 0.35) (layer "F.Cu") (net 4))
 (segment (start 96.711782 93.33122) (end 110.7 92.9) (width 0.35) (layer "F.Cu") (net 4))
 (segment (start 142.9 97.2) (end 144.9 97.2) (width 0.35) (layer "F.Cu") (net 4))
 (segment (start 95.75 97.5) (end 96 97.05) (width 0.35) (layer "F.Cu") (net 4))
 (segment (start 76.4 100.85) (end 77.7 101.15) (width 0.35) (layer "F.Cu") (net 4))
 (segment (start 132 94.9) (end 141.9 96.95) (width 0.35) (layer "F.Cu") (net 4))
 (segment (start 149.04 98.44) (end 154.35 98.15) (width 0.35) (layer "F.Cu") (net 14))
 (segment (start 154.35 98.15) (end 164.977407 94.471897) (width 0.35) (layer "F.Cu") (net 14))
 (segment (start 149.04 95.9) (end 154.25 95.2) (width 0.35) (layer "F.Cu") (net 13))
 (segment (start 154.25 95.2) (end 164.320006 92.018445) (width 0.35) (layer "F.Cu") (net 13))
 (segment (start 208.4 95.3) (end 217.6 96.25) (width 0.35) (layer "B.Cu") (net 12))
 (segment (start 197.75 94.45) (end 204.65 94.85) (width 0.35) (layer "B.Cu") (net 12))
 (segment (start 204.65 94.85) (end 208.4 95.3) (width 0.35) (layer "B.Cu") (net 12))
 (segment (start 217.6 96.25) (end 219.5 96.05) (width 0.35) (layer "B.Cu") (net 12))
 (segment (start 219.5 96.05) (end 220.911581 94.725183) (width 0.35) (layer "B.Cu") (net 12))
 (segment (start 196.7 94.15) (end 197.75 94.45) (width 0.35) (layer "B.Cu") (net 12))
 (segment (start 195.600469 92.783813) (end 196.7 94.15) (width 0.35) (layer "B.Cu") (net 12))
 (segment (start 213.25 90) (end 215.95 90.05) (width 0.35) (layer "B.Cu") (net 11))
 (segment (start 215.95 90.05) (end 219.2 90.35) (width 0.35) (layer "B.Cu") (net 11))
 (segment (start 219.2 90.35) (end 221.088762 92.19137) (width 0.35) (layer "B.Cu") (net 11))
 (segment (start 198.134281 92.960994) (end 213.25 90) (width 0.35) (layer "B.Cu") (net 11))
 (segment (start 197.15 89.45) (end 197 90.85) (width 0.35) (layer "F.Cu") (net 8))
 (segment (start 199 91.75) (end 215.843955 94.37082) (width 0.35) (layer "F.Cu") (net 8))
 (segment (start 197.2 91.4) (end 197.85 91.7) (width 0.35) (layer "F.Cu") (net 8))
 (segment (start 195.954831 87.716188) (end 197.15 89.45) (width 0.35) (layer "F.Cu") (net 8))
 (segment (start 197 90.85) (end 197.2 91.4) (width 0.35) (layer "F.Cu") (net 8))
 (segment (start 197.85 91.7) (end 199 91.75) (width 0.35) (layer "F.Cu") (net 8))
 (segment (start 196.85 92.05) (end 196.825469 93.25) (width 0.35) (layer "F.Cu") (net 10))
 (segment (start 196.825469 93.25) (end 197.15 94.15) (width 0.35) (layer "F.Cu") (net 10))
 (segment (start 211.7 95.75) (end 216.55 96.3) (width 0.35) (layer "F.Cu") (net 10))
 (segment (start 195.77765 90.25) (end 196.85 92.05) (width 0.35) (layer "F.Cu") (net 10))
 (segment (start 198.05 94.4) (end 203.95 94.75) (width 0.35) (layer "F.Cu") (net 10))
 (segment (start 197.15 94.15) (end 198.05 94.4) (width 0.35) (layer "F.Cu") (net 10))
 (segment (start 203.95 94.75) (end 211.7 95.75) (width 0.35) (layer "F.Cu") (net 10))
 (segment (start 216.55 96.3) (end 218.377768 94.548001) (width 0.35) (layer "F.Cu") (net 10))
 (segment (start 216.95 93.2) (end 218.55495 92.014189) (width 0.35) (layer "F.Cu") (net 9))
 (segment (start 198.311463 90.427182) (end 214.45 93) (width 0.35) (layer "F.Cu") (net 9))
 (segment (start 214.45 93) (end 216.95 93.2) (width 0.35) (layer "F.Cu") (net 9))
 (segment (start 198.488644 87.893369) (end 216.021137 91.837007) (width 0.35) (layer "F.Cu") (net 7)))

